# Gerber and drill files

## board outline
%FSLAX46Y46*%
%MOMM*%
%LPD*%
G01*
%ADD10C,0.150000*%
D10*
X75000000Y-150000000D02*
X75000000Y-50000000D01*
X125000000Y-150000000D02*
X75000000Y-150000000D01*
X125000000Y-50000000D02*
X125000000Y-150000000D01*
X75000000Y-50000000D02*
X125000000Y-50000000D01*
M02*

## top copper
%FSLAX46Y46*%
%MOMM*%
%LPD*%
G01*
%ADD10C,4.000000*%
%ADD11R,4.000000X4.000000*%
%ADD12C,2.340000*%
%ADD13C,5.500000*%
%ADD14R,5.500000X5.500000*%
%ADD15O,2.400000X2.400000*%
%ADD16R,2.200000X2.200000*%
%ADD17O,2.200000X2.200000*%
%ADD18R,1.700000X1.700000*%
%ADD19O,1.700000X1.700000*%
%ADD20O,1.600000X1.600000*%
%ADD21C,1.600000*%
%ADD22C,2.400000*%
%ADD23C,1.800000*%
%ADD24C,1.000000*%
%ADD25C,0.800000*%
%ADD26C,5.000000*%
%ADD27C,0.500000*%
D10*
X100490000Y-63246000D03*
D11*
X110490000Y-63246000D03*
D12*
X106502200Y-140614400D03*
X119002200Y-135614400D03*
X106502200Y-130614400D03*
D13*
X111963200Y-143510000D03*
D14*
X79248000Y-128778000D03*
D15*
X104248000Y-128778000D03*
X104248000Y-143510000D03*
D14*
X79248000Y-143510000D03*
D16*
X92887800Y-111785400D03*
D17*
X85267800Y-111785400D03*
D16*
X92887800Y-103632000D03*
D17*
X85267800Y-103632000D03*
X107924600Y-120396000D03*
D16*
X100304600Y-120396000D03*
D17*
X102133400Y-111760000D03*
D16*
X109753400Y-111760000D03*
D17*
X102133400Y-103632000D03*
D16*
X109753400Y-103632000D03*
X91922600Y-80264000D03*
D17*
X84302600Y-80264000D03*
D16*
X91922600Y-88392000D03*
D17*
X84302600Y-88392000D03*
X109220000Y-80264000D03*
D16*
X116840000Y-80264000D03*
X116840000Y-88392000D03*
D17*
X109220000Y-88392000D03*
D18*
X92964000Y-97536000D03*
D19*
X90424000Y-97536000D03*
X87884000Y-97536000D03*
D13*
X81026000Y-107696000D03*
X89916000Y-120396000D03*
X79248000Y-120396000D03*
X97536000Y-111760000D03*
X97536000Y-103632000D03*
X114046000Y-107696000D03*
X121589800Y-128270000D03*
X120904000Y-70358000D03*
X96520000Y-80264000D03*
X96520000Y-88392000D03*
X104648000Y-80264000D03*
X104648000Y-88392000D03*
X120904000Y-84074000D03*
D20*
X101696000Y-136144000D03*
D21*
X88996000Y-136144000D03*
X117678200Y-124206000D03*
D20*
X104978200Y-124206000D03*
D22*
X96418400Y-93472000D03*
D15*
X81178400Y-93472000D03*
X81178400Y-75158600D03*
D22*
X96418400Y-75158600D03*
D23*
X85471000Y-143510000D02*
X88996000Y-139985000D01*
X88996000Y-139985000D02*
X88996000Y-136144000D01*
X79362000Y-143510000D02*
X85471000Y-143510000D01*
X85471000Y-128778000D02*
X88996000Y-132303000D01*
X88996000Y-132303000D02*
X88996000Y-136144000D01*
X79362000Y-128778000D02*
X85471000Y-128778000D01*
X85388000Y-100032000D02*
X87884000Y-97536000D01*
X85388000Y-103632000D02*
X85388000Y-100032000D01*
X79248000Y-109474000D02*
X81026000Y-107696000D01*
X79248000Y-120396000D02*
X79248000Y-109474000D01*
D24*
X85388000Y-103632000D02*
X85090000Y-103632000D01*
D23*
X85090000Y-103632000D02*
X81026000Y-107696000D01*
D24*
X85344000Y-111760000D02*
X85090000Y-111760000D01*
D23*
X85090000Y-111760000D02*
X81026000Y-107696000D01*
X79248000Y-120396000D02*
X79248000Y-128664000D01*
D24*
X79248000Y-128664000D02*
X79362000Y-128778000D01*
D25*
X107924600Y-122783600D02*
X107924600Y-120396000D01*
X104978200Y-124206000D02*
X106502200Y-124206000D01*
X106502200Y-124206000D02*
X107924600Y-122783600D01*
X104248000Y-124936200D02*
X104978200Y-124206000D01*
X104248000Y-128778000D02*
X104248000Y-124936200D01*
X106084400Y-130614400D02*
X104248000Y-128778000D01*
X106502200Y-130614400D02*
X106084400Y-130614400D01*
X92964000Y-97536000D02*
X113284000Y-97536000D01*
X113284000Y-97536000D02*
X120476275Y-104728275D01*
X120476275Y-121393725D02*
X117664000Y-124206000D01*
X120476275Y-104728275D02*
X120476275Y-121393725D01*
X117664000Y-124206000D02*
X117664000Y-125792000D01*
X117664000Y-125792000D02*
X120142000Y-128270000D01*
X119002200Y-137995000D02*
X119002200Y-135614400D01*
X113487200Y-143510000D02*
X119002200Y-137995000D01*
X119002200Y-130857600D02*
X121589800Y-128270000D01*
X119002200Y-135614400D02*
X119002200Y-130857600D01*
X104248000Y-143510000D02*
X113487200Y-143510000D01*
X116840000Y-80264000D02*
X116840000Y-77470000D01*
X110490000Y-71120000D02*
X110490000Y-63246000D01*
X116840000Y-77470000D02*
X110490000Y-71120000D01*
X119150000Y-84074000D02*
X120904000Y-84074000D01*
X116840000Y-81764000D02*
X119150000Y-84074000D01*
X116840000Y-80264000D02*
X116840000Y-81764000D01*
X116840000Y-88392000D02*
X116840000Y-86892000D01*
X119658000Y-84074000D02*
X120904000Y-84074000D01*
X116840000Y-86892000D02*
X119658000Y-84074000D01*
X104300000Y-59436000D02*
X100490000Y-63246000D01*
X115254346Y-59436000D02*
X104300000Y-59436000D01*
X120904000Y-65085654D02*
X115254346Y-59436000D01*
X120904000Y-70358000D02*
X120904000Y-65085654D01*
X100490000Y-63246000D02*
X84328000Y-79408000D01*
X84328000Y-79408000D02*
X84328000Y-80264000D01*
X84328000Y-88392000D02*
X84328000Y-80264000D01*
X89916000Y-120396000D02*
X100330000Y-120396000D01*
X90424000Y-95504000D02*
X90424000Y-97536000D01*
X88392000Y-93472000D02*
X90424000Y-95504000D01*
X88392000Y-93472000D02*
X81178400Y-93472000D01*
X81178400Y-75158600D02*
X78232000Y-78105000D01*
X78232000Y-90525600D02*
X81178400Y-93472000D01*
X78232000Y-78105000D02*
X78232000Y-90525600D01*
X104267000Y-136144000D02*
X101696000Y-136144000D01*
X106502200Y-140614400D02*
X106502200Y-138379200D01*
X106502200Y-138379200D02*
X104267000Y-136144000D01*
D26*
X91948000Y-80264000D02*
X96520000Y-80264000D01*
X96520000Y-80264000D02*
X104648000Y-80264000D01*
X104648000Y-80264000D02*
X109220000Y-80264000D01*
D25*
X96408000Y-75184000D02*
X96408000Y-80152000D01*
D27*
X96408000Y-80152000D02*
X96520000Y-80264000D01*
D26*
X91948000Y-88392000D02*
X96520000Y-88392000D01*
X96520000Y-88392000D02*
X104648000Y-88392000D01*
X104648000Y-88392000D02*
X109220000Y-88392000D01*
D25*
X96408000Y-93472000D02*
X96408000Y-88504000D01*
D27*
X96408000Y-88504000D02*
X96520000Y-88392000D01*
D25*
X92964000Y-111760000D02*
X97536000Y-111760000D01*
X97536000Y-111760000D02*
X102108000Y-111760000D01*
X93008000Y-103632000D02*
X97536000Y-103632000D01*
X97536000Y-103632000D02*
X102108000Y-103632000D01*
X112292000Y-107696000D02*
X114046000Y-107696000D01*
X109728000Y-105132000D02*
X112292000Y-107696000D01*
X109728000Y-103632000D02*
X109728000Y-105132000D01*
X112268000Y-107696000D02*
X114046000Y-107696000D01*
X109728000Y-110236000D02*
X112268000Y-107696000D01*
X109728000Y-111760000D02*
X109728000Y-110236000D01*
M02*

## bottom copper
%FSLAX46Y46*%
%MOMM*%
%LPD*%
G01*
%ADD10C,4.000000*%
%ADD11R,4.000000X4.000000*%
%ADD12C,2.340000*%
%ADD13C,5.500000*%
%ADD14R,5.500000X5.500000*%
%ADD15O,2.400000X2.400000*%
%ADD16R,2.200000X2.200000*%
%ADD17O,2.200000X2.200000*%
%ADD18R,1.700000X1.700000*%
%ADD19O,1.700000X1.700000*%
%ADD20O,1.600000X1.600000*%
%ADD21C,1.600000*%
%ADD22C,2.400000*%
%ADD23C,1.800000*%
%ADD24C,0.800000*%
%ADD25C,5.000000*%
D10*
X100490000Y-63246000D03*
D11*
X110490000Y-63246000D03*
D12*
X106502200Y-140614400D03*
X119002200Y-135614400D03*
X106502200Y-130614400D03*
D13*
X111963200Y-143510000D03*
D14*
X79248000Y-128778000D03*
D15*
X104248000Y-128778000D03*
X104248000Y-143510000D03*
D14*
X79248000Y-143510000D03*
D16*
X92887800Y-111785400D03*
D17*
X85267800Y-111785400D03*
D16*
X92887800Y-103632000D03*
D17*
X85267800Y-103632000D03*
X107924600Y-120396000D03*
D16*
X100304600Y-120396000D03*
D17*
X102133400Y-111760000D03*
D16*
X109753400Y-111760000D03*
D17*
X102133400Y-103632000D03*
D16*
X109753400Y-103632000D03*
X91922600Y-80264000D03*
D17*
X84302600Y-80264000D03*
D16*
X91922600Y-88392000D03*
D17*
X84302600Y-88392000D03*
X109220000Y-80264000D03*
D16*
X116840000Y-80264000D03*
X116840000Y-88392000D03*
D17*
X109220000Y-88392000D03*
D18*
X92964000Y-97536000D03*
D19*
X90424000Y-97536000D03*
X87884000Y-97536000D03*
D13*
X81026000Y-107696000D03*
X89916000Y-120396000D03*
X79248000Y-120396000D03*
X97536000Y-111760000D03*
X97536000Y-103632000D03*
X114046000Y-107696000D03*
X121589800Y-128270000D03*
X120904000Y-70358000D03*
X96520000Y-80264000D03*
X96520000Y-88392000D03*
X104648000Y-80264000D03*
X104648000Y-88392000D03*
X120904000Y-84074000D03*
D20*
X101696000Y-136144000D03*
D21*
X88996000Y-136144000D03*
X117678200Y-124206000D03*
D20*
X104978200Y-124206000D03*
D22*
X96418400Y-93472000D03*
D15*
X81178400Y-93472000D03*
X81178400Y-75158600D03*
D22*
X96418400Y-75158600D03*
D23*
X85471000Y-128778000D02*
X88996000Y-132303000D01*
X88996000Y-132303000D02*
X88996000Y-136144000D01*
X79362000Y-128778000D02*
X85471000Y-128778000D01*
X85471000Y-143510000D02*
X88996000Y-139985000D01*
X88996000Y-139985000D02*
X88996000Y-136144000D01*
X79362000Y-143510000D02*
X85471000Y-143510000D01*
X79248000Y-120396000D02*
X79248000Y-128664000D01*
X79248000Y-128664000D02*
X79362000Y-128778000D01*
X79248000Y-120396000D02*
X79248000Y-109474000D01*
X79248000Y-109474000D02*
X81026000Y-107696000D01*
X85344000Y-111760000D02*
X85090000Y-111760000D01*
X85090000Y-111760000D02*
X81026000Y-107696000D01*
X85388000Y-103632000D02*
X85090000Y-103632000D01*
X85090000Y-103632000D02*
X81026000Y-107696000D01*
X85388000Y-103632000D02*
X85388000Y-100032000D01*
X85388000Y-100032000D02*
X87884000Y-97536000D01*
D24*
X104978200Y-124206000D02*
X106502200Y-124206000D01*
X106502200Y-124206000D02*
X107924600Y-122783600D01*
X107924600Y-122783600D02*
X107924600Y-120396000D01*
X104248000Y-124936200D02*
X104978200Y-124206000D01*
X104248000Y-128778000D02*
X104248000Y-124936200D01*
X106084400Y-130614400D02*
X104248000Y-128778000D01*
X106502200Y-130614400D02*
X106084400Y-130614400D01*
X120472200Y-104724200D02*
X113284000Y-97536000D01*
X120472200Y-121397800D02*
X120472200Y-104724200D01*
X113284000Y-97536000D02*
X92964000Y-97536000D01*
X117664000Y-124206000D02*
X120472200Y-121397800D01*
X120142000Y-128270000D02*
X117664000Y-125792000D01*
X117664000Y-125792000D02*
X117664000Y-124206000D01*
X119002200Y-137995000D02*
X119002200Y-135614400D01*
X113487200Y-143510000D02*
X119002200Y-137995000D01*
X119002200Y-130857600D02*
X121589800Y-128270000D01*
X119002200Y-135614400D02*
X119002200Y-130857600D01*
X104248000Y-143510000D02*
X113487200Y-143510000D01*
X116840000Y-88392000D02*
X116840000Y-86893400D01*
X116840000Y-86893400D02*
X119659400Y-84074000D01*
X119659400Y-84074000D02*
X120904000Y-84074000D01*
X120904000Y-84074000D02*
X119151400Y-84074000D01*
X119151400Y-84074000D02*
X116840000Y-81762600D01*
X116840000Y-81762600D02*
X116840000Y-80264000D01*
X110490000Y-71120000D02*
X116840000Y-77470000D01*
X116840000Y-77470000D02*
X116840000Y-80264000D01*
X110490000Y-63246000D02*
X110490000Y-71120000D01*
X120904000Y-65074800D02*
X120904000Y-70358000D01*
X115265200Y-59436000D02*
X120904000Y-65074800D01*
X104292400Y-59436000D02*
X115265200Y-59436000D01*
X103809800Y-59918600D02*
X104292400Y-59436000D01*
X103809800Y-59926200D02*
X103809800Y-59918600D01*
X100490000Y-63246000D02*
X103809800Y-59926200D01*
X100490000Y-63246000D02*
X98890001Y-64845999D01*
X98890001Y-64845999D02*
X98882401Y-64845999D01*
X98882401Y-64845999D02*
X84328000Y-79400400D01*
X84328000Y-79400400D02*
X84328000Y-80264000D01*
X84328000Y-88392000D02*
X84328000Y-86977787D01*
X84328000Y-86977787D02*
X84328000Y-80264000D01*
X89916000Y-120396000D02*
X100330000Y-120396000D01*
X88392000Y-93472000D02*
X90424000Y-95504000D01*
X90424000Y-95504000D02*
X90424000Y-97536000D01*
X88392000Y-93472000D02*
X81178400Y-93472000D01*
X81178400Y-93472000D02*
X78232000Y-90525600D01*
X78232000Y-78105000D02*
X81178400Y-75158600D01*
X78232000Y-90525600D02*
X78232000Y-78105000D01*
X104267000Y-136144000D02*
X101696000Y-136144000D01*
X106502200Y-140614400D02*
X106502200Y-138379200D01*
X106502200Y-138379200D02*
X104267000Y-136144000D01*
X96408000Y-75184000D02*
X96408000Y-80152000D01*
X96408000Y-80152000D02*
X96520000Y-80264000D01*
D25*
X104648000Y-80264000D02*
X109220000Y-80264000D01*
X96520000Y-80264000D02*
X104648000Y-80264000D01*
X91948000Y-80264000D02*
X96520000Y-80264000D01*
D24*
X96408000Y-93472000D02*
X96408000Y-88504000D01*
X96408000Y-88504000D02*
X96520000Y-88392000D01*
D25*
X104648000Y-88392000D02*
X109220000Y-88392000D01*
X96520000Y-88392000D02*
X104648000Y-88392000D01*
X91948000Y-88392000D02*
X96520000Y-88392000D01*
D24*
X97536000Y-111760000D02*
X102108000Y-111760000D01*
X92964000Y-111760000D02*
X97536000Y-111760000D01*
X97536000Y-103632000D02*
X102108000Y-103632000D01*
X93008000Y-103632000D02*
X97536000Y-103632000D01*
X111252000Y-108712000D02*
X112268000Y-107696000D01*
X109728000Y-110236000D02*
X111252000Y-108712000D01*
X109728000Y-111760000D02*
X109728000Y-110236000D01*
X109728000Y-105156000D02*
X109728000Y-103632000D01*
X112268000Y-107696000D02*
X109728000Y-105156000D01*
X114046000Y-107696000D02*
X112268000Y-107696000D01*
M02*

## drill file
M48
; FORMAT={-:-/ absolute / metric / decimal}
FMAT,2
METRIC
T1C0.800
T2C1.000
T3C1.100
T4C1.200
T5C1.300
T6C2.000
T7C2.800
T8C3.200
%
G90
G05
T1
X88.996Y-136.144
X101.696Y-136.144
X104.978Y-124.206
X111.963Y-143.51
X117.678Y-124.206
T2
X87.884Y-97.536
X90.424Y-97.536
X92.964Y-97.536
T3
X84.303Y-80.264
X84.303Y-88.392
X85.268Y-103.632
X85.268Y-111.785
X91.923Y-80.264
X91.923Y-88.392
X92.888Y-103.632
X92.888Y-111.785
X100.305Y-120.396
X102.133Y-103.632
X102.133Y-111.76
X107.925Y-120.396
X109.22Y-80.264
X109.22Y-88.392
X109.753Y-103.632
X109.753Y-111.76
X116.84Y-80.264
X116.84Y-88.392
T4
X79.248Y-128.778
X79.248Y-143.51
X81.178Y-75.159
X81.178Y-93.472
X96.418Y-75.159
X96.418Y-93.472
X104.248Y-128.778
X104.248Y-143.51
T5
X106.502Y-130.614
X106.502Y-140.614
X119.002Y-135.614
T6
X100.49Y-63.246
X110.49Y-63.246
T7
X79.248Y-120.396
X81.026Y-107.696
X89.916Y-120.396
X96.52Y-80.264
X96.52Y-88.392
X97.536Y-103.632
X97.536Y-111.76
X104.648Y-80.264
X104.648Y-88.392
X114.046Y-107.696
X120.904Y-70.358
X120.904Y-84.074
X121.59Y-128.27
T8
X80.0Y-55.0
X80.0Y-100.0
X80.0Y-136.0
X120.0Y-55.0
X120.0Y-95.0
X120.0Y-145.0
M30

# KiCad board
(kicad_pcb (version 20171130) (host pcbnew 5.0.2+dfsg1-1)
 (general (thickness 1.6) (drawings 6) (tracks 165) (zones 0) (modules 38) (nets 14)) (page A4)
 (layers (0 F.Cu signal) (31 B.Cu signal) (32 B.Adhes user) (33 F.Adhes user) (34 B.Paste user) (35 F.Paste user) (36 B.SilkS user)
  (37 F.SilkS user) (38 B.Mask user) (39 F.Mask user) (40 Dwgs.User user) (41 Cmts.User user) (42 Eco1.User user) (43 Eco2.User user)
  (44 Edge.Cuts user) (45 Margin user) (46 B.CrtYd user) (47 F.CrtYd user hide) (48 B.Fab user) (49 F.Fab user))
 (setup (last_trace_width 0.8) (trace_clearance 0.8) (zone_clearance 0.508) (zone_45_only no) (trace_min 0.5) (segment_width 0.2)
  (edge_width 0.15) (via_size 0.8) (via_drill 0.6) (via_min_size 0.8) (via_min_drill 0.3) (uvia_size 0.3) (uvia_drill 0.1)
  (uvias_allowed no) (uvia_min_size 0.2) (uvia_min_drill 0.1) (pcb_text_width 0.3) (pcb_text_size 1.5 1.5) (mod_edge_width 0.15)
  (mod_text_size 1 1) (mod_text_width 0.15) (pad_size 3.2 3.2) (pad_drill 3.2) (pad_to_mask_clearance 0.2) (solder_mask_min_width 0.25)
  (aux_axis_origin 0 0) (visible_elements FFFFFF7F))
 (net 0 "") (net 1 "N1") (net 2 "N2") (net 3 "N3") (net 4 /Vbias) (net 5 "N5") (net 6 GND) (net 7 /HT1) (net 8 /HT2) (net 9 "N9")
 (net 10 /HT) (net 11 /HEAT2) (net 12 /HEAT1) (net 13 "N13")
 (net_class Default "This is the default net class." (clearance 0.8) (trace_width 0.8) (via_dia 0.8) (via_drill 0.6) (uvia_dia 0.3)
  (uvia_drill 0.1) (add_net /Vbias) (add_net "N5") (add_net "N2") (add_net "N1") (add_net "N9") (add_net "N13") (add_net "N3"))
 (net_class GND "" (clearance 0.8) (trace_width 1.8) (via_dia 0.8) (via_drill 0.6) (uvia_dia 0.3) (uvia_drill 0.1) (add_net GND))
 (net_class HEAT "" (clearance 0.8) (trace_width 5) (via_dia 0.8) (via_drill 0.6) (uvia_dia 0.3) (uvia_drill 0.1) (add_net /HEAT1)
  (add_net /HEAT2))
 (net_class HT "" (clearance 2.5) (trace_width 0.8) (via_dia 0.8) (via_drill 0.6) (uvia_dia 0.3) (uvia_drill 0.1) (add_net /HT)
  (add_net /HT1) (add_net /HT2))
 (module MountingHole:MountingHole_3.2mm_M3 (layer F.Cu) (at 80 136)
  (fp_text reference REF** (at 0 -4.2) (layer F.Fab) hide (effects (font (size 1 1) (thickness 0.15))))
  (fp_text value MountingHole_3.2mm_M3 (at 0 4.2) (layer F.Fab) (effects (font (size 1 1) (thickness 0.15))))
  (pad "" np_thru_hole circle (at 0 0) (size 3.2 3.2) (drill 3.2) (layers *.Cu *.Mask) (clearance 2)))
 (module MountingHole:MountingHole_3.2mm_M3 (layer F.Cu) (at 120 145)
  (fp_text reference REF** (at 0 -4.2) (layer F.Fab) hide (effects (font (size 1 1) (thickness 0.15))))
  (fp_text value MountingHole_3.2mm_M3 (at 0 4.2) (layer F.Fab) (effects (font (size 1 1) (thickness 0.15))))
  (pad "" np_thru_hole circle (at 0 0) (size 3.2 3.2) (drill 3.2) (layers *.Cu *.Mask) (clearance 2)))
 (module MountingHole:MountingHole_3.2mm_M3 (layer F.Cu) (at 80 55)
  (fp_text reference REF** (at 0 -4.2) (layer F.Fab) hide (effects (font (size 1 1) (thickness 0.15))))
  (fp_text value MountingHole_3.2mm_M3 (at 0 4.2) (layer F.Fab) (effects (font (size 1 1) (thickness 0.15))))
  (pad "" np_thru_hole circle (at 0 0) (size 3.2 3.2) (drill 3.2) (layers *.Cu *.Mask) (clearance 2)))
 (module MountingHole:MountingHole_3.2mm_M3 (layer F.Cu) (at 120 55)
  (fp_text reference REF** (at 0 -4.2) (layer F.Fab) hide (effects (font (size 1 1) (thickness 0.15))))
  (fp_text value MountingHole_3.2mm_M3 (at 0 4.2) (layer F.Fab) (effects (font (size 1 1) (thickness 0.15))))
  (pad "" np_thru_hole circle (at 0 0) (size 3.2 3.2) (drill 3.2) (layers *.Cu *.Mask) (clearance 2)))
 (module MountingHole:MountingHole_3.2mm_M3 (layer F.Cu) (at 120 95)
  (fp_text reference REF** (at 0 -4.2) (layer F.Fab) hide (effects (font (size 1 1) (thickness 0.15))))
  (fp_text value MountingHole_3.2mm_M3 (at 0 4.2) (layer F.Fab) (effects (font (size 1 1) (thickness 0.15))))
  (pad "" np_thru_hole circle (at 0 0) (size 3.2 3.2) (drill 3.2) (layers *.Cu *.Mask) (clearance 2)))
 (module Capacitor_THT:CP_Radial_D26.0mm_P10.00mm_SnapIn (layer F.Cu) (at 110.49 63.246 180)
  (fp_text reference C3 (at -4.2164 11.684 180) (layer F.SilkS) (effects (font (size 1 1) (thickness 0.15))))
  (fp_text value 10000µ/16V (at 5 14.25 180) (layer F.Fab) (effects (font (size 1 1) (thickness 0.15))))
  (pad 2 thru_hole circle (at 10 0 180) (size 4 4) (drill 2) (layers *.Cu *.Mask) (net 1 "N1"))
  (pad 1 thru_hole rect (at 0 0 180) (size 4 4) (drill 2) (layers *.Cu *.Mask) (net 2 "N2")))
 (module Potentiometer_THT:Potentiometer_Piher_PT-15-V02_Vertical (layer F.Cu) (at 106.5022 140.6144)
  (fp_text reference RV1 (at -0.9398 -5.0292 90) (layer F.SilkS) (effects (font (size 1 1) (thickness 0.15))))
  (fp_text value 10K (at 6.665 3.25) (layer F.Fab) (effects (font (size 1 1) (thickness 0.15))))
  (pad 1 thru_hole circle (at 0 0) (size 2.34 2.34) (drill 1.3) (layers *.Cu *.Mask) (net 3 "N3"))
  (pad 2 thru_hole circle (at 12.5 -5) (size 2.34 2.34) (drill 1.3) (layers *.Cu *.Mask) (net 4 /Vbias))
  (pad 3 thru_hole circle (at 0 -10) (size 2.34 2.34) (drill 1.3) (layers *.Cu *.Mask) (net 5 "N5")))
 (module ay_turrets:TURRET (layer F.Cu) (at 111.9632 143.51)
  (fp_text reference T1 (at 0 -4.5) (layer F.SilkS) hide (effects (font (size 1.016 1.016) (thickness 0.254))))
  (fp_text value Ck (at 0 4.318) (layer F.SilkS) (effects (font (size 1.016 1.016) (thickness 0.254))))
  (pad 1 thru_hole circle (at 0 0) (size 5.5 5.5) (drill 0.8) (layers *.Cu *.Mask F.SilkS) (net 4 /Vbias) (clearance 0.5)))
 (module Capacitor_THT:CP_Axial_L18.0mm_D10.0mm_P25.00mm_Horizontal (layer F.Cu) (at 79.248 128.778)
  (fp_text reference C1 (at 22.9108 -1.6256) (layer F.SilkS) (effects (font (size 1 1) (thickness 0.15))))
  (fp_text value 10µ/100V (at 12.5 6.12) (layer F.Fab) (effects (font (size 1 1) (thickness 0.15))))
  (pad 1 thru_hole rect (at 0 0) (size 5.5 5.5) (drill 1.2) (layers *.Cu *.Mask) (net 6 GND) (clearance 0.5))
  (pad 2 thru_hole oval (at 25 0) (size 2.4 2.4) (drill 1.2) (layers *.Cu *.Mask) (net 5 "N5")))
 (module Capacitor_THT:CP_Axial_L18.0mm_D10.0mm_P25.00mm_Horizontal (layer F.Cu) (at 79.248 143.51)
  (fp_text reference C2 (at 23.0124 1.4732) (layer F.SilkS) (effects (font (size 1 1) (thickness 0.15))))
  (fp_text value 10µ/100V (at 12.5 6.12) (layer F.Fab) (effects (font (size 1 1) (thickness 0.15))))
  (pad 2 thru_hole oval (at 25 0) (size 2.4 2.4) (drill 1.2) (layers *.Cu *.Mask) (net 4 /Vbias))
  (pad 1 thru_hole rect (at 0 0) (size 5.5 5.5) (drill 1.2) (layers *.Cu *.Mask) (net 6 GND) (clearance 0.5)))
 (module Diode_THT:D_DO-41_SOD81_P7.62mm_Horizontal (layer F.Cu) (at 92.8878 111.7854 180)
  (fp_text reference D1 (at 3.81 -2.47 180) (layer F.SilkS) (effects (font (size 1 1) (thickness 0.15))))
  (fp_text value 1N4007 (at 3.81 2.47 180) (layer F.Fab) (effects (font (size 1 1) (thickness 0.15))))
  (pad 1 thru_hole rect (at 0 0 180) (size 2.2 2.2) (drill 1.1) (layers *.Cu *.Mask) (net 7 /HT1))
  (pad 2 thru_hole oval (at 7.62 0 180) (size 2.2 2.2) (drill 1.1) (layers *.Cu *.Mask) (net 6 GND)))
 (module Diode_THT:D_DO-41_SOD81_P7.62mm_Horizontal (layer F.Cu) (at 92.8878 103.632 180)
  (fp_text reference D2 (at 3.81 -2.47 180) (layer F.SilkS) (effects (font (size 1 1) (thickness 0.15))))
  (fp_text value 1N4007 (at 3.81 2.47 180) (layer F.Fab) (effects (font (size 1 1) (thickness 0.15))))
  (pad 1 thru_hole rect (at 0 0 180) (size 2.2 2.2) (drill 1.1) (layers *.Cu *.Mask) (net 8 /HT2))
  (pad 2 thru_hole oval (at 7.62 0 180) (size 2.2 2.2) (drill 1.1) (layers *.Cu *.Mask) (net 6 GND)))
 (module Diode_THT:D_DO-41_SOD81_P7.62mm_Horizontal (layer F.Cu) (at 100.3046 120.396)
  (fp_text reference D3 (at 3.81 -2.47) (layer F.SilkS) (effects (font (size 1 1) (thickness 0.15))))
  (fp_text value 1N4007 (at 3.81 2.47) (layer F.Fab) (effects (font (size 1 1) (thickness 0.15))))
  (pad 2 thru_hole oval (at 7.62 0) (size 2.2 2.2) (drill 1.1) (layers *.Cu *.Mask) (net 5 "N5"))
  (pad 1 thru_hole rect (at 0 0) (size 2.2 2.2) (drill 1.1) (layers *.Cu *.Mask) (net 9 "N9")))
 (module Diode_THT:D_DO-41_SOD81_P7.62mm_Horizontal (layer F.Cu) (at 109.7534 111.76 180)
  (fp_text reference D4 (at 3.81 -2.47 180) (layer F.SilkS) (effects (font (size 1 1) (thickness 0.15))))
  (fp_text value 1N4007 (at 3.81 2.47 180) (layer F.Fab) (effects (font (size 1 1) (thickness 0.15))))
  (pad 2 thru_hole oval (at 7.62 0 180) (size 2.2 2.2) (drill 1.1) (layers *.Cu *.Mask) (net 7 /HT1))
  (pad 1 thru_hole rect (at 0 0 180) (size 2.2 2.2) (drill 1.1) (layers *.Cu *.Mask) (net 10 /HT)))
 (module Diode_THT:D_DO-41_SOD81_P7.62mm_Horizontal (layer F.Cu) (at 109.7534 103.632 180)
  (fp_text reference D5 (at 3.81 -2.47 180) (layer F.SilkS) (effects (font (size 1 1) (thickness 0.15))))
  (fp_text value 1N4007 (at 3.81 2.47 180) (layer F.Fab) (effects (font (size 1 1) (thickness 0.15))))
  (pad 2 thru_hole oval (at 7.62 0 180) (size 2.2 2.2) (drill 1.1) (layers *.Cu *.Mask) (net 8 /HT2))
  (pad 1 thru_hole rect (at 0 0 180) (size 2.2 2.2) (drill 1.1) (layers *.Cu *.Mask) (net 10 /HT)))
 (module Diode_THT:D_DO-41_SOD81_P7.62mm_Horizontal (layer F.Cu) (at 91.9226 80.264 180)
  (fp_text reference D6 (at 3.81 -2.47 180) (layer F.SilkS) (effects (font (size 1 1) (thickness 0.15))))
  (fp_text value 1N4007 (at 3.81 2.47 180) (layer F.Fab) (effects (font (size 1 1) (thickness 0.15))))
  (pad 1 thru_hole rect (at 0 0 180) (size 2.2 2.2) (drill 1.1) (layers *.Cu *.Mask) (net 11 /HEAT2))
  (pad 2 thru_hole oval (at 7.62 0 180) (size 2.2 2.2) (drill 1.1) (layers *.Cu *.Mask) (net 1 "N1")))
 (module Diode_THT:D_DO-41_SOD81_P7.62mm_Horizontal (layer F.Cu) (at 91.9226 88.392 180)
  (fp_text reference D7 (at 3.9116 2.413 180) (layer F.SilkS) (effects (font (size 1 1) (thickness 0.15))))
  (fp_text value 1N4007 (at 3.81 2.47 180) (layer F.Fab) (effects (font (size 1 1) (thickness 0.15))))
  (pad 1 thru_hole rect (at 0 0 180) (size 2.2 2.2) (drill 1.1) (layers *.Cu *.Mask) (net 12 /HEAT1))
  (pad 2 thru_hole oval (at 7.62 0 180) (size 2.2 2.2) (drill 1.1) (layers *.Cu *.Mask) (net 1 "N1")))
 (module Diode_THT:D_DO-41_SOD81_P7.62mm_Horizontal (layer F.Cu) (at 116.84 80.264 180)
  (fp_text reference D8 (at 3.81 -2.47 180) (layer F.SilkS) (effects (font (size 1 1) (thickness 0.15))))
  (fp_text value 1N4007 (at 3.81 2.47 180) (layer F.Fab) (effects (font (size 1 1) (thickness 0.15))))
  (pad 2 thru_hole oval (at 7.62 0 180) (size 2.2 2.2) (drill 1.1) (layers *.Cu *.Mask) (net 11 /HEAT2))
  (pad 1 thru_hole rect (at 0 0 180) (size 2.2 2.2) (drill 1.1) (layers *.Cu *.Mask) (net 2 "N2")))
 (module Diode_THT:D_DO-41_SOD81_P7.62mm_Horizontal (layer F.Cu) (at 116.84 88.392 180)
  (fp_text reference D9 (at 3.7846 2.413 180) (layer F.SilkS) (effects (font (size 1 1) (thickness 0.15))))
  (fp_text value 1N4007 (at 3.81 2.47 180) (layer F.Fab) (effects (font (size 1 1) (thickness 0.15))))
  (pad 1 thru_hole rect (at 0 0 180) (size 2.2 2.2) (drill 1.1) (layers *.Cu *.Mask) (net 2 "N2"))
  (pad 2 thru_hole oval (at 7.62 0 180) (size 2.2 2.2) (drill 1.1) (layers *.Cu *.Mask) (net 12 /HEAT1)))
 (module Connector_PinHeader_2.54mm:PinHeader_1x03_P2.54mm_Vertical (layer F.Cu) (at 92.964 97.536 270)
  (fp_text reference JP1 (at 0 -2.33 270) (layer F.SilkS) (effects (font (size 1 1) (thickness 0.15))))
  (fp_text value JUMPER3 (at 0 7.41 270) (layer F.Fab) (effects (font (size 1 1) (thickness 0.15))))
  (pad 1 thru_hole rect (at 0 0 270) (size 1.7 1.7) (drill 1) (layers *.Cu *.Mask) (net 4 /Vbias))
  (pad 2 thru_hole oval (at 0 2.54 270) (size 1.7 1.7) (drill 1) (layers *.Cu *.Mask) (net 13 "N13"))
  (pad 3 thru_hole oval (at 0 5.08 270) (size 1.7 1.7) (drill 1) (layers *.Cu *.Mask) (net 6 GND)))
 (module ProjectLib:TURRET (layer F.Cu) (at 81.026 107.696)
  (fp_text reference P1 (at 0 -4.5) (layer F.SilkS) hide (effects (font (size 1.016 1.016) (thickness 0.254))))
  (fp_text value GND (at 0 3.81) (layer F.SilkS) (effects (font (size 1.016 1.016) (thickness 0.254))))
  (pad 1 thru_hole circle (at 0 0) (size 5.5 5.5) (drill 2.8) (layers *.Cu *.Mask F.SilkS) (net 6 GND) (clearance 0.5)))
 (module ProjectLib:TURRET (layer F.Cu) (at 89.916 120.396)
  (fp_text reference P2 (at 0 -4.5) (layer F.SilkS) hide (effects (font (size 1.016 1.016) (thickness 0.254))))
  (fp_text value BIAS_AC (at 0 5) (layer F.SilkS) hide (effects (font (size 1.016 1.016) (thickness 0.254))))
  (pad 1 thru_hole circle (at 0 0) (size 5.5 5.5) (drill 2.8) (layers *.Cu *.Mask F.SilkS) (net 9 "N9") (clearance 0.5)))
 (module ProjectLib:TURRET (layer F.Cu) (at 79.248 120.396)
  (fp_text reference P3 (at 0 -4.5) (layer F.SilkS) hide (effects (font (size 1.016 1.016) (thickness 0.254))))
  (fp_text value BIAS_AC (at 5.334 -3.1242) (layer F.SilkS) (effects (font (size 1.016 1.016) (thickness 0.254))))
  (pad 1 thru_hole circle (at 0 0) (size 5.5 5.5) (drill 2.8) (layers *.Cu *.Mask F.SilkS) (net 6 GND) (clearance 0.5)))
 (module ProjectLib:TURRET (layer F.Cu) (at 97.536 111.76)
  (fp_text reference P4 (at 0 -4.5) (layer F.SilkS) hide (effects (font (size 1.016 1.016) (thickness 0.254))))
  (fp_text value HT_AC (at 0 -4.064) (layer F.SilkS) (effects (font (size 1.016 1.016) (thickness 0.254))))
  (pad 1 thru_hole circle (at 0 0) (size 5.5 5.5) (drill 2.8) (layers *.Cu *.Mask F.SilkS) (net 7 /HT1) (clearance 0.5)))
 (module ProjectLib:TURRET (layer F.Cu) (at 97.536 103.632)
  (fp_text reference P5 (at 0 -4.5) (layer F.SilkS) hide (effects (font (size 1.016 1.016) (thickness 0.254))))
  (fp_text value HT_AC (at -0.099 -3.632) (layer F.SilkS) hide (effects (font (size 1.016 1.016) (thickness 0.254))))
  (pad 1 thru_hole circle (at 0 0) (size 5.5 5.5) (drill 2.8) (layers *.Cu *.Mask F.SilkS) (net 8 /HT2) (clearance 0.5)))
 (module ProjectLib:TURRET (layer F.Cu) (at 114.046 107.696)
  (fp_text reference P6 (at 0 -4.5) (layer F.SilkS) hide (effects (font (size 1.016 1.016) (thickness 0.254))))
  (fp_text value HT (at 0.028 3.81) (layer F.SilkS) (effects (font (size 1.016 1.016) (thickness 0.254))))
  (pad 1 thru_hole circle (at 0 0) (size 5.5 5.5) (drill 2.8) (layers *.Cu *.Mask F.SilkS) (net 10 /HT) (clearance 0.5)))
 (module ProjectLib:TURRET (layer F.Cu) (at 121.5898 128.27)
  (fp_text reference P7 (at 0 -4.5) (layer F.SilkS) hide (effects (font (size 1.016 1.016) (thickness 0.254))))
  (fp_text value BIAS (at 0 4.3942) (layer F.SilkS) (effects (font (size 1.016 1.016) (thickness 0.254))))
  (pad 1 thru_hole circle (at 0 0) (size 5.5 5.5) (drill 2.8) (layers *.Cu *.Mask F.SilkS) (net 4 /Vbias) (clearance 0.5)))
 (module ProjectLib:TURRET (layer F.Cu) (at 120.904 70.358)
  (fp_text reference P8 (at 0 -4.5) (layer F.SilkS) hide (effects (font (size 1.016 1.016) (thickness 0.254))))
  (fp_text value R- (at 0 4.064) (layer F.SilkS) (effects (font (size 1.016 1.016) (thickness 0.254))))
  (pad 1 thru_hole circle (at 0 0) (size 5.5 5.5) (drill 2.8) (layers *.Cu *.Mask F.SilkS) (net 1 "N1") (clearance 0.5)))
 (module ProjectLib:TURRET (layer F.Cu) (at 96.52 80.264)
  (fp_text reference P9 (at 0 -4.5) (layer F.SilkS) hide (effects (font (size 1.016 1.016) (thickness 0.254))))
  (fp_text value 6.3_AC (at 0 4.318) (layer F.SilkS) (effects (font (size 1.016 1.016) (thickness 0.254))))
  (pad 1 thru_hole circle (at 0 0) (size 5.5 5.5) (drill 2.8) (layers *.Cu *.Mask F.SilkS) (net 11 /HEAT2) (clearance 0.5)))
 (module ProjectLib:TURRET (layer F.Cu) (at 96.52 88.392)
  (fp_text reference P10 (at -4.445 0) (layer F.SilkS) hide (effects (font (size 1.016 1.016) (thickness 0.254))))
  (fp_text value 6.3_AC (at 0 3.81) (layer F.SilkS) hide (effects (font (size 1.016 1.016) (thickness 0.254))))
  (pad 1 thru_hole circle (at 0 0) (size 5.5 5.5) (drill 2.8) (layers *.Cu *.Mask F.SilkS) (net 12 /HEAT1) (clearance 0.5)))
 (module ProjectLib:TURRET (layer F.Cu) (at 104.648 80.264)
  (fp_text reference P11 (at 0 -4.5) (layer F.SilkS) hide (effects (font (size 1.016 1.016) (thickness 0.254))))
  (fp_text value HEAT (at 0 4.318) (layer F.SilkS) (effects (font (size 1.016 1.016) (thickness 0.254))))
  (pad 1 thru_hole circle (at 0 0) (size 5.5 5.5) (drill 2.8) (layers *.Cu *.Mask F.SilkS) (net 11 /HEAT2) (clearance 0.5)))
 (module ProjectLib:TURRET (layer F.Cu) (at 104.648 88.392)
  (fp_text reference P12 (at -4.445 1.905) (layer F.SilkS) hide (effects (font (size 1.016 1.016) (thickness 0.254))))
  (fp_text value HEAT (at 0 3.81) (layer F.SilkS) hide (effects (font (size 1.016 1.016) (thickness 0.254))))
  (pad 1 thru_hole circle (at 0 0) (size 5.5 5.5) (drill 2.8) (layers *.Cu *.Mask F.SilkS) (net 12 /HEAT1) (clearance 0.5)))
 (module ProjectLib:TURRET (layer F.Cu) (at 120.904 84.074)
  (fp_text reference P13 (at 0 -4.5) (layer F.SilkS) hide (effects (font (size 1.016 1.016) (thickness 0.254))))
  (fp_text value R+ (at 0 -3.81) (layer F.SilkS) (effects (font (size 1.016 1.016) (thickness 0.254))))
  (pad 1 thru_hole circle (at 0 0) (size 5.5 5.5) (drill 2.8) (layers *.Cu *.Mask F.SilkS) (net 2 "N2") (clearance 0.5)))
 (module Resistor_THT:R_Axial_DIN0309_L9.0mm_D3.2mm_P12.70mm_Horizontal (layer F.Cu) (at 88.996 136.144)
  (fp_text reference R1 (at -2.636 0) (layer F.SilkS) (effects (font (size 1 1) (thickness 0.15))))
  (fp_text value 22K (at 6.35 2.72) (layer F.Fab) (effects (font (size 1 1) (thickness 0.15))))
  (pad 2 thru_hole oval (at 12.7 0) (size 1.6 1.6) (drill 0.8) (layers *.Cu *.Mask) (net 3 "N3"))
  (pad 1 thru_hole circle (at 0 0) (size 1.6 1.6) (drill 0.8) (layers *.Cu *.Mask) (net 6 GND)))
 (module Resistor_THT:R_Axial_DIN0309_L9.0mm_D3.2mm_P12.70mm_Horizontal (layer F.Cu) (at 117.6782 124.206 180)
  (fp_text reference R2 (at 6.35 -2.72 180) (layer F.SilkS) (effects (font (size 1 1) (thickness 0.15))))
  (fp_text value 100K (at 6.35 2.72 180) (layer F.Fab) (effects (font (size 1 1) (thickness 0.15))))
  (pad 1 thru_hole circle (at 0 0 180) (size 1.6 1.6) (drill 0.8) (layers *.Cu *.Mask) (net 4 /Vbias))
  (pad 2 thru_hole oval (at 12.7 0 180) (size 1.6 1.6) (drill 0.8) (layers *.Cu *.Mask) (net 5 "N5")))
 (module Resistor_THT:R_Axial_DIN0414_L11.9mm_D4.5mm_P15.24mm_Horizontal (layer F.Cu) (at 96.4184 93.472 180)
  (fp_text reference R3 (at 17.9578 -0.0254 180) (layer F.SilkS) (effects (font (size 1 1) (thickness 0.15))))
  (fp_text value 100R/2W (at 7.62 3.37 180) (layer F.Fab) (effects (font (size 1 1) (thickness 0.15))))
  (pad 1 thru_hole circle (at 0 0 180) (size 2.4 2.4) (drill 1.2) (layers *.Cu *.Mask) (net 12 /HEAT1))
  (pad 2 thru_hole oval (at 15.24 0 180) (size 2.4 2.4) (drill 1.2) (layers *.Cu *.Mask) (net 13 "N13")))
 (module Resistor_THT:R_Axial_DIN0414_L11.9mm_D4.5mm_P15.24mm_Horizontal (layer F.Cu) (at 96.4184 75.1586 180)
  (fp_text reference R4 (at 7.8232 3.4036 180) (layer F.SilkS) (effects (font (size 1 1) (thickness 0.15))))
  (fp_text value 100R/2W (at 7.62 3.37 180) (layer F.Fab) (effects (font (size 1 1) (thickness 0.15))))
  (pad 2 thru_hole oval (at 15.24 0 180) (size 2.4 2.4) (drill 1.2) (layers *.Cu *.Mask) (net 13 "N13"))
  (pad 1 thru_hole circle (at 0 0 180) (size 2.4 2.4) (drill 1.2) (layers *.Cu *.Mask) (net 11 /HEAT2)))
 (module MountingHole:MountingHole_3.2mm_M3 (layer F.Cu) (at 80 100)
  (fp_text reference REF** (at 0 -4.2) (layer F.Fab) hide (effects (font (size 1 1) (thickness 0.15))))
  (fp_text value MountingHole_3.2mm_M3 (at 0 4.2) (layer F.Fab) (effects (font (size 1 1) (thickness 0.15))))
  (pad "" np_thru_hole circle (at 0 0) (size 3.2 3.2) (drill 3.2) (layers *.Cu *.Mask) (clearance 2)))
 (gr_line (start 75 150) (end 75 50) (layer Edge.Cuts) (width 0.15))
 (gr_line (start 125 150) (end 75 150) (layer Edge.Cuts) (width 0.15))
 (gr_line (start 125 50) (end 125 150) (layer Edge.Cuts) (width 0.15))
 (gr_line (start 75 50) (end 125 50) (layer Edge.Cuts) (width 0.15))
 (segment (start 85.471 128.778) (end 88.996 132.303) (width 1.8) (layer B.Cu) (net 6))
 (segment (start 88.996 132.303) (end 88.996 136.144) (width 1.8) (layer B.Cu) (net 6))
 (segment (start 79.362 128.778) (end 85.471 128.778) (width 1.8) (layer B.Cu) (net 6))
 (segment (start 85.471 143.51) (end 88.996 139.985) (width 1.8) (layer B.Cu) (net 6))
 (segment (start 88.996 139.985) (end 88.996 136.144) (width 1.8) (layer B.Cu) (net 6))
 (segment (start 79.362 143.51) (end 85.471 143.51) (width 1.8) (layer B.Cu) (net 6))
 (segment (start 85.471 143.51) (end 88.996 139.985) (width 1.8) (layer F.Cu) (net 6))
 (segment (start 88.996 139.985) (end 88.996 136.144) (width 1.8) (layer F.Cu) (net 6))
 (segment (start 79.362 143.51) (end 85.471 143.51) (width 1.8) (layer F.Cu) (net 6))
 (segment (start 85.471 128.778) (end 88.996 132.303) (width 1.8) (layer F.Cu) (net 6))
 (segment (start 88.996 132.303) (end 88.996 136.144) (width 1.8) (layer F.Cu) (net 6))
 (segment (start 79.362 128.778) (end 85.471 128.778) (width 1.8) (layer F.Cu) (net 6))
 (segment (start 79.248 120.396) (end 79.248 128.664) (width 1.8) (layer B.Cu) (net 6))
 (segment (start 79.248 128.664) (end 79.362 128.778) (width 1.8) (layer B.Cu) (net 6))
 (segment (start 79.248 120.396) (end 79.248 109.474) (width 1.8) (layer B.Cu) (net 6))
 (segment (start 79.248 109.474) (end 81.026 107.696) (width 1.8) (layer B.Cu) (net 6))
 (segment (start 85.344 111.76) (end 85.09 111.76) (width 1.8) (layer B.Cu) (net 6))
 (segment (start 85.09 111.76) (end 81.026 107.696) (width 1.8) (layer B.Cu) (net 6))
 (segment (start 85.388 103.632) (end 85.09 103.632) (width 1.8) (layer B.Cu) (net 6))
 (segment (start 85.09 103.632) (end 81.026 107.696) (width 1.8) (layer B.Cu) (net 6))
 (segment (start 85.388 103.632) (end 85.388 100.032) (width 1.8) (layer B.Cu) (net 6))
 (segment (start 85.388 100.032) (end 87.884 97.536) (width 1.8) (layer B.Cu) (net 6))
 (segment (start 85.388 100.032) (end 87.884 97.536) (width 1.8) (layer F.Cu) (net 6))
 (segment (start 85.388 103.632) (end 85.388 100.032) (width 1.8) (layer F.Cu) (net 6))
 (segment (start 79.248 109.474) (end 81.026 107.696) (width 1.8) (layer F.Cu) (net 6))
 (segment (start 79.248 120.396) (end 79.248 109.474) (width 1.8) (layer F.Cu) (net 6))
 (segment (start 85.388 103.632) (end 85.09 103.632) (width 1) (layer F.Cu) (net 6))
 (segment (start 85.09 103.632) (end 81.026 107.696) (width 1.8) (layer F.Cu) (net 6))
 (segment (start 85.344 111.76) (end 85.09 111.76) (width 1) (layer F.Cu) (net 6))
 (segment (start 85.09 111.76) (end 81.026 107.696) (width 1.8) (layer F.Cu) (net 6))
 (segment (start 79.248 120.396) (end 79.248 128.664) (width 1.8) (layer F.Cu) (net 6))
 (segment (start 79.248 128.664) (end 79.362 128.778) (width 1) (layer F.Cu) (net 6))
 (segment (start 107.9246 122.7836) (end 107.9246 120.396) (width 0.8) (layer F.Cu) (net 5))
 (segment (start 104.9782 124.206) (end 106.5022 124.206) (width 0.8) (layer F.Cu) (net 5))
 (segment (start 106.5022 124.206) (end 107.9246 122.7836) (width 0.8) (layer F.Cu) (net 5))
 (segment (start 104.9782 124.206) (end 106.5022 124.206) (width 0.8) (layer B.Cu) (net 5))
 (segment (start 106.5022 124.206) (end 107.9246 122.7836) (width 0.8) (layer B.Cu) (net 5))
 (segment (start 107.9246 122.7836) (end 107.9246 120.396) (width 0.8) (layer B.Cu) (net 5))
 (segment (start 104.248 124.9362) (end 104.9782 124.206) (width 0.8) (layer F.Cu) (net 5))
 (segment (start 104.248 128.778) (end 104.248 124.9362) (width 0.8) (layer F.Cu) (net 5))
 (segment (start 106.0844 130.6144) (end 104.248 128.778) (width 0.8) (layer F.Cu) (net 5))
 (segment (start 106.5022 130.6144) (end 106.0844 130.6144) (width 0.8) (layer F.Cu) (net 5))
 (segment (start 104.248 124.9362) (end 104.9782 124.206) (width 0.8) (layer B.Cu) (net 5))
 (segment (start 104.248 128.778) (end 104.248 124.9362) (width 0.8) (layer B.Cu) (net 5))
 (segment (start 106.0844 130.6144) (end 104.248 128.778) (width 0.8) (layer B.Cu) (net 5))
 (segment (start 106.5022 130.6144) (end 106.0844 130.6144) (width 0.8) (layer B.Cu) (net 5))
 (segment (start 92.964 97.536) (end 113.284 97.536) (width 0.8) (layer F.Cu) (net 4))
 (segment (start 113.284 97.536) (end 120.476275 104.728275) (width 0.8) (layer F.Cu) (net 4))
 (segment (start 120.476275 121.393725) (end 117.664 124.206) (width 0.8) (layer F.Cu) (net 4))
 (segment (start 120.476275 104.728275) (end 120.476275 121.393725) (width 0.8) (layer F.Cu) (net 4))
 (segment (start 117.664 124.206) (end 117.664 125.792) (width 0.8) (layer F.Cu) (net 4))
 (segment (start 117.664 125.792) (end 120.142 128.27) (width 0.8) (layer F.Cu) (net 4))
 (segment (start 120.4722 104.7242) (end 113.284 97.536) (width 0.8) (layer B.Cu) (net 4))
 (segment (start 120.4722 121.3978) (end 120.4722 104.7242) (width 0.8) (layer B.Cu) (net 4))
 (segment (start 113.284 97.536) (end 92.964 97.536) (width 0.8) (layer B.Cu) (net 4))
 (segment (start 117.664 124.206) (end 120.4722 121.3978) (width 0.8) (layer B.Cu) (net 4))
 (segment (start 120.142 128.27) (end 117.664 125.792) (width 0.8) (layer B.Cu) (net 4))
 (segment (start 117.664 125.792) (end 117.664 124.206) (width 0.8) (layer B.Cu) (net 4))
 (segment (start 119.0022 137.995) (end 119.0022 135.6144) (width 0.8) (layer B.Cu) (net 4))
 (segment (start 113.4872 143.51) (end 119.0022 137.995) (width 0.8) (layer B.Cu) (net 4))
 (segment (start 119.0022 130.8576) (end 121.5898 128.27) (width 0.8) (layer B.Cu) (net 4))
 (segment (start 119.0022 135.6144) (end 119.0022 130.8576) (width 0.8) (layer B.Cu) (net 4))
 (segment (start 119.0022 137.995) (end 119.0022 135.6144) (width 0.8) (layer F.Cu) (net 4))
 (segment (start 113.4872 143.51) (end 119.0022 137.995) (width 0.8) (layer F.Cu) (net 4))
 (segment (start 119.0022 130.8576) (end 121.5898 128.27) (width 0.8) (layer F.Cu) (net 4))
 (segment (start 119.0022 135.6144) (end 119.0022 130.8576) (width 0.8) (layer F.Cu) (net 4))
 (segment (start 104.248 143.51) (end 113.4872 143.51) (width 0.8) (layer B.Cu) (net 4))
 (segment (start 104.248 143.51) (end 113.4872 143.51) (width 0.8) (layer F.Cu) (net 4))
 (segment (start 116.84 88.392) (end 116.84 86.8934) (width 0.8) (layer B.Cu) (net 2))
 (segment (start 116.84 86.8934) (end 119.6594 84.074) (width 0.8) (layer B.Cu) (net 2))
 (segment (start 119.6594 84.074) (end 120.904 84.074) (width 0.8) (layer B.Cu) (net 2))
 (segment (start 120.904 84.074) (end 119.1514 84.074) (width 0.8) (layer B.Cu) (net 2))
 (segment (start 119.1514 84.074) (end 116.84 81.7626) (width 0.8) (layer B.Cu) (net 2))
 (segment (start 116.84 81.7626) (end 116.84 80.264) (width 0.8) (layer B.Cu) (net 2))
 (segment (start 110.49 71.12) (end 116.84 77.47) (width 0.8) (layer B.Cu) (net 2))
 (segment (start 116.84 77.47) (end 116.84 80.264) (width 0.8) (layer B.Cu) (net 2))
 (segment (start 110.49 63.246) (end 110.49 71.12) (width 0.8) (layer B.Cu) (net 2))
 (segment (start 116.84 80.264) (end 116.84 77.47) (width 0.8) (layer F.Cu) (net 2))
 (segment (start 110.49 71.12) (end 110.49 63.246) (width 0.8) (layer F.Cu) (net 2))
 (segment (start 116.84 77.47) (end 110.49 71.12) (width 0.8) (layer F.Cu) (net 2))
 (segment (start 119.15 84.074) (end 120.904 84.074) (width 0.8) (layer F.Cu) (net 2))
 (segment (start 116.84 81.764) (end 119.15 84.074) (width 0.8) (layer F.Cu) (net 2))
 (segment (start 116.84 80.264) (end 116.84 81.764) (width 0.8) (layer F.Cu) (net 2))
 (segment (start 116.84 88.392) (end 116.84 86.892) (width 0.8) (layer F.Cu) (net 2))
 (segment (start 119.658 84.074) (end 120.904 84.074) (width 0.8) (layer F.Cu) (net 2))
 (segment (start 116.84 86.892) (end 119.658 84.074) (width 0.8) (layer F.Cu) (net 2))
 (segment (start 120.904 65.0748) (end 120.904 70.358) (width 0.8) (layer B.Cu) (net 1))
 (segment (start 115.2652 59.436) (end 120.904 65.0748) (width 0.8) (layer B.Cu) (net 1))
 (segment (start 104.2924 59.436) (end 115.2652 59.436) (width 0.8) (layer B.Cu) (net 1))
 (segment (start 103.8098 59.9186) (end 104.2924 59.436) (width 0.8) (layer B.Cu) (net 1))
 (segment (start 103.8098 59.9262) (end 103.8098 59.9186) (width 0.8) (layer B.Cu) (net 1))
 (segment (start 100.49 63.246) (end 103.8098 59.9262) (width 0.8) (layer B.Cu) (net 1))
 (segment (start 100.49 63.246) (end 98.890001 64.845999) (width 0.8) (layer B.Cu) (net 1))
 (segment (start 98.890001 64.845999) (end 98.882401 64.845999) (width 0.8) (layer B.Cu) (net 1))
 (segment (start 98.882401 64.845999) (end 84.328 79.4004) (width 0.8) (layer B.Cu) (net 1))
 (segment (start 84.328 79.4004) (end 84.328 80.264) (width 0.8) (layer B.Cu) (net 1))
 (segment (start 84.328 88.392) (end 84.328 86.977787) (width 0.8) (layer B.Cu) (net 1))
 (segment (start 84.328 86.977787) (end 84.328 80.264) (width 0.8) (layer B.Cu) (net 1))
 (segment (start 104.3 59.436) (end 100.49 63.246) (width 0.8) (layer F.Cu) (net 1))
 (segment (start 115.254346 59.436) (end 104.3 59.436) (width 0.8) (layer F.Cu) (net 1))
 (segment (start 120.904 65.085654) (end 115.254346 59.436) (width 0.8) (layer F.Cu) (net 1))
 (segment (start 120.904 70.358) (end 120.904 65.085654) (width 0.8) (layer F.Cu) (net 1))
 (segment (start 100.49 63.246) (end 84.328 79.408) (width 0.8) (layer F.Cu) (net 1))
 (segment (start 84.328 79.408) (end 84.328 80.264) (width 0.8) (layer F.Cu) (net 1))
 (segment (start 84.328 88.392) (end 84.328 80.264) (width 0.8) (layer F.Cu) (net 1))
 (segment (start 89.916 120.396) (end 100.33 120.396) (width 0.8) (layer B.Cu) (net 9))
 (segment (start 89.916 120.396) (end 100.33 120.396) (width 0.8) (layer F.Cu) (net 9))
 (segment (start 88.392 93.472) (end 90.424 95.504) (width 0.8) (layer B.Cu) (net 13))
 (segment (start 90.424 95.504) (end 90.424 97.536) (width 0.8) (layer B.Cu) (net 13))
 (segment (start 90.424 95.504) (end 90.424 97.536) (width 0.8) (layer F.Cu) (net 13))
 (segment (start 88.392 93.472) (end 90.424 95.504) (width 0.8) (layer F.Cu) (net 13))
 (segment (start 88.392 93.472) (end 81.1784 93.472) (width 0.8) (layer F.Cu) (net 13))
 (segment (start 88.392 93.472) (end 81.1784 93.472) (width 0.8) (layer B.Cu) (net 13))
 (segment (start 81.1784 93.472) (end 78.232 90.5256) (width 0.8) (layer B.Cu) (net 13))
 (segment (start 78.232 78.105) (end 81.1784 75.1586) (width 0.8) (layer B.Cu) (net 13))
 (segment (start 78.232 90.5256) (end 78.232 78.105) (width 0.8) (layer B.Cu) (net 13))
 (segment (start 81.1784 75.1586) (end 78.232 78.105) (width 0.8) (layer F.Cu) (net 13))
 (segment (start 78.232 90.5256) (end 81.1784 93.472) (width 0.8) (layer F.Cu) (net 13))
 (segment (start 78.232 78.105) (end 78.232 90.5256) (width 0.8) (layer F.Cu) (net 13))
 (segment (start 104.267 136.144) (end 101.696 136.144) (width 0.8) (layer F.Cu) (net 3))
 (segment (start 106.5022 140.6144) (end 106.5022 138.3792) (width 0.8) (layer F.Cu) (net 3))
 (segment (start 106.5022 138.3792) (end 104.267 136.144) (width 0.8) (layer F.Cu) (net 3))
 (segment (start 104.267 136.144) (end 101.696 136.144) (width 0.8) (layer B.Cu) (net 3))
 (segment (start 106.5022 140.6144) (end 106.5022 138.3792) (width 0.8) (layer B.Cu) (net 3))
 (segment (start 106.5022 138.3792) (end 104.267 136.144) (width 0.8) (layer B.Cu) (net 3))
 (segment (start 96.408 75.184) (end 96.408 80.152) (width 0.8) (layer B.Cu) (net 11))
 (segment (start 96.408 80.152) (end 96.52 80.264) (width 0.8) (layer B.Cu) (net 11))
 (segment (start 104.648 80.264) (end 109.22 80.264) (width 5) (layer B.Cu) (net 11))
 (segment (start 96.52 80.264) (end 104.648 80.264) (width 5) (layer B.Cu) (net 11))
 (segment (start 91.948 80.264) (end 96.52 80.264) (width 5) (layer B.Cu) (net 11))
 (segment (start 91.948 80.264) (end 96.52 80.264) (width 5) (layer F.Cu) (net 11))
 (segment (start 96.52 80.264) (end 104.648 80.264) (width 5) (layer F.Cu) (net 11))
 (segment (start 104.648 80.264) (end 109.22 80.264) (width 5) (layer F.Cu) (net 11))
 (segment (start 96.408 75.184) (end 96.408 80.152) (width 0.8) (layer F.Cu) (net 11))
 (segment (start 96.408 80.152) (end 96.52 80.264) (width 0.5) (layer F.Cu) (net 11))
 (segment (start 96.408 93.472) (end 96.408 88.504) (width 0.8) (layer B.Cu) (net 12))
 (segment (start 96.408 88.504) (end 96.52 88.392) (width 0.8) (layer B.Cu) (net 12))
 (segment (start 104.648 88.392) (end 109.22 88.392) (width 5) (layer B.Cu) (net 12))
 (segment (start 96.52 88.392) (end 104.648 88.392) (width 5) (layer B.Cu) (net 12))
 (segment (start 91.948 88.392) (end 96.52 88.392) (width 5) (layer B.Cu) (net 12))
 (segment (start 91.948 88.392) (end 96.52 88.392) (width 5) (layer F.Cu) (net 12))
 (segment (start 96.52 88.392) (end 104.648 88.392) (width 5) (layer F.Cu) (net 12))
 (segment (start 104.648 88.392) (end 109.22 88.392) (width 5) (layer F.Cu) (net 12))
 (segment (start 96.408 93.472) (end 96.408 88.504) (width 0.8) (layer F.Cu) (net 12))
 (segment (start 96.408 88.504) (end 96.52 88.392) (width 0.5) (layer F.Cu) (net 12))
 (segment (start 97.536 111.76) (end 102.108 111.76) (width 0.8) (layer B.Cu) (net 7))
 (segment (start 92.964 111.76) (end 97.536 111.76) (width 0.8) (layer B.Cu) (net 7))
 (segment (start 92.964 111.76) (end 97.536 111.76) (width 0.8) (layer F.Cu) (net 7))
 (segment (start 97.536 111.76) (end 102.108 111.76) (width 0.8) (layer F.Cu) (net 7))
 (segment (start 97.536 103.632) (end 102.108 103.632) (width 0.8) (layer B.Cu) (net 8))
 (segment (start 93.008 103.632) (end 97.536 103.632) (width 0.8) (layer B.Cu) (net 8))
 (segment (start 93.008 103.632) (end 97.536 103.632) (width 0.8) (layer F.Cu) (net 8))
 (segment (start 97.536 103.632) (end 102.108 103.632) (width 0.8) (layer F.Cu) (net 8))
 (segment (start 111.252 108.712) (end 112.268 107.696) (width 0.8) (layer B.Cu) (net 10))
 (segment (start 109.728 110.236) (end 111.252 108.712) (width 0.8) (layer B.Cu) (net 10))
 (segment (start 109.728 111.76) (end 109.728 110.236) (width 0.8) (layer B.Cu) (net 10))
 (segment (start 109.728 105.156) (end 109.728 103.632) (width 0.8) (layer B.Cu) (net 10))
 (segment (start 112.268 107.696) (end 109.728 105.156) (width 0.8) (layer B.Cu) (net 10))
 (segment (start 114.046 107.696) (end 112.268 107.696) (width 0.8) (layer B.Cu) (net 10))
 (segment (start 112.292 107.696) (end 114.046 107.696) (width 0.8) (layer F.Cu) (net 10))
 (segment (start 109.728 105.132) (end 112.292 107.696) (width 0.8) (layer F.Cu) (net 10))
 (segment (start 109.728 103.632) (end 109.728 105.132) (width 0.8) (layer F.Cu) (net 10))
 (segment (start 112.268 107.696) (end 114.046 107.696) (width 0.8) (layer F.Cu) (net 10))
 (segment (start 109.728 110.236) (end 112.268 107.696) (width 0.8) (layer F.Cu) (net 10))
 (segment (start 109.728 111.76) (end 109.728 110.236) (width 0.8) (layer F.Cu) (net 10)))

